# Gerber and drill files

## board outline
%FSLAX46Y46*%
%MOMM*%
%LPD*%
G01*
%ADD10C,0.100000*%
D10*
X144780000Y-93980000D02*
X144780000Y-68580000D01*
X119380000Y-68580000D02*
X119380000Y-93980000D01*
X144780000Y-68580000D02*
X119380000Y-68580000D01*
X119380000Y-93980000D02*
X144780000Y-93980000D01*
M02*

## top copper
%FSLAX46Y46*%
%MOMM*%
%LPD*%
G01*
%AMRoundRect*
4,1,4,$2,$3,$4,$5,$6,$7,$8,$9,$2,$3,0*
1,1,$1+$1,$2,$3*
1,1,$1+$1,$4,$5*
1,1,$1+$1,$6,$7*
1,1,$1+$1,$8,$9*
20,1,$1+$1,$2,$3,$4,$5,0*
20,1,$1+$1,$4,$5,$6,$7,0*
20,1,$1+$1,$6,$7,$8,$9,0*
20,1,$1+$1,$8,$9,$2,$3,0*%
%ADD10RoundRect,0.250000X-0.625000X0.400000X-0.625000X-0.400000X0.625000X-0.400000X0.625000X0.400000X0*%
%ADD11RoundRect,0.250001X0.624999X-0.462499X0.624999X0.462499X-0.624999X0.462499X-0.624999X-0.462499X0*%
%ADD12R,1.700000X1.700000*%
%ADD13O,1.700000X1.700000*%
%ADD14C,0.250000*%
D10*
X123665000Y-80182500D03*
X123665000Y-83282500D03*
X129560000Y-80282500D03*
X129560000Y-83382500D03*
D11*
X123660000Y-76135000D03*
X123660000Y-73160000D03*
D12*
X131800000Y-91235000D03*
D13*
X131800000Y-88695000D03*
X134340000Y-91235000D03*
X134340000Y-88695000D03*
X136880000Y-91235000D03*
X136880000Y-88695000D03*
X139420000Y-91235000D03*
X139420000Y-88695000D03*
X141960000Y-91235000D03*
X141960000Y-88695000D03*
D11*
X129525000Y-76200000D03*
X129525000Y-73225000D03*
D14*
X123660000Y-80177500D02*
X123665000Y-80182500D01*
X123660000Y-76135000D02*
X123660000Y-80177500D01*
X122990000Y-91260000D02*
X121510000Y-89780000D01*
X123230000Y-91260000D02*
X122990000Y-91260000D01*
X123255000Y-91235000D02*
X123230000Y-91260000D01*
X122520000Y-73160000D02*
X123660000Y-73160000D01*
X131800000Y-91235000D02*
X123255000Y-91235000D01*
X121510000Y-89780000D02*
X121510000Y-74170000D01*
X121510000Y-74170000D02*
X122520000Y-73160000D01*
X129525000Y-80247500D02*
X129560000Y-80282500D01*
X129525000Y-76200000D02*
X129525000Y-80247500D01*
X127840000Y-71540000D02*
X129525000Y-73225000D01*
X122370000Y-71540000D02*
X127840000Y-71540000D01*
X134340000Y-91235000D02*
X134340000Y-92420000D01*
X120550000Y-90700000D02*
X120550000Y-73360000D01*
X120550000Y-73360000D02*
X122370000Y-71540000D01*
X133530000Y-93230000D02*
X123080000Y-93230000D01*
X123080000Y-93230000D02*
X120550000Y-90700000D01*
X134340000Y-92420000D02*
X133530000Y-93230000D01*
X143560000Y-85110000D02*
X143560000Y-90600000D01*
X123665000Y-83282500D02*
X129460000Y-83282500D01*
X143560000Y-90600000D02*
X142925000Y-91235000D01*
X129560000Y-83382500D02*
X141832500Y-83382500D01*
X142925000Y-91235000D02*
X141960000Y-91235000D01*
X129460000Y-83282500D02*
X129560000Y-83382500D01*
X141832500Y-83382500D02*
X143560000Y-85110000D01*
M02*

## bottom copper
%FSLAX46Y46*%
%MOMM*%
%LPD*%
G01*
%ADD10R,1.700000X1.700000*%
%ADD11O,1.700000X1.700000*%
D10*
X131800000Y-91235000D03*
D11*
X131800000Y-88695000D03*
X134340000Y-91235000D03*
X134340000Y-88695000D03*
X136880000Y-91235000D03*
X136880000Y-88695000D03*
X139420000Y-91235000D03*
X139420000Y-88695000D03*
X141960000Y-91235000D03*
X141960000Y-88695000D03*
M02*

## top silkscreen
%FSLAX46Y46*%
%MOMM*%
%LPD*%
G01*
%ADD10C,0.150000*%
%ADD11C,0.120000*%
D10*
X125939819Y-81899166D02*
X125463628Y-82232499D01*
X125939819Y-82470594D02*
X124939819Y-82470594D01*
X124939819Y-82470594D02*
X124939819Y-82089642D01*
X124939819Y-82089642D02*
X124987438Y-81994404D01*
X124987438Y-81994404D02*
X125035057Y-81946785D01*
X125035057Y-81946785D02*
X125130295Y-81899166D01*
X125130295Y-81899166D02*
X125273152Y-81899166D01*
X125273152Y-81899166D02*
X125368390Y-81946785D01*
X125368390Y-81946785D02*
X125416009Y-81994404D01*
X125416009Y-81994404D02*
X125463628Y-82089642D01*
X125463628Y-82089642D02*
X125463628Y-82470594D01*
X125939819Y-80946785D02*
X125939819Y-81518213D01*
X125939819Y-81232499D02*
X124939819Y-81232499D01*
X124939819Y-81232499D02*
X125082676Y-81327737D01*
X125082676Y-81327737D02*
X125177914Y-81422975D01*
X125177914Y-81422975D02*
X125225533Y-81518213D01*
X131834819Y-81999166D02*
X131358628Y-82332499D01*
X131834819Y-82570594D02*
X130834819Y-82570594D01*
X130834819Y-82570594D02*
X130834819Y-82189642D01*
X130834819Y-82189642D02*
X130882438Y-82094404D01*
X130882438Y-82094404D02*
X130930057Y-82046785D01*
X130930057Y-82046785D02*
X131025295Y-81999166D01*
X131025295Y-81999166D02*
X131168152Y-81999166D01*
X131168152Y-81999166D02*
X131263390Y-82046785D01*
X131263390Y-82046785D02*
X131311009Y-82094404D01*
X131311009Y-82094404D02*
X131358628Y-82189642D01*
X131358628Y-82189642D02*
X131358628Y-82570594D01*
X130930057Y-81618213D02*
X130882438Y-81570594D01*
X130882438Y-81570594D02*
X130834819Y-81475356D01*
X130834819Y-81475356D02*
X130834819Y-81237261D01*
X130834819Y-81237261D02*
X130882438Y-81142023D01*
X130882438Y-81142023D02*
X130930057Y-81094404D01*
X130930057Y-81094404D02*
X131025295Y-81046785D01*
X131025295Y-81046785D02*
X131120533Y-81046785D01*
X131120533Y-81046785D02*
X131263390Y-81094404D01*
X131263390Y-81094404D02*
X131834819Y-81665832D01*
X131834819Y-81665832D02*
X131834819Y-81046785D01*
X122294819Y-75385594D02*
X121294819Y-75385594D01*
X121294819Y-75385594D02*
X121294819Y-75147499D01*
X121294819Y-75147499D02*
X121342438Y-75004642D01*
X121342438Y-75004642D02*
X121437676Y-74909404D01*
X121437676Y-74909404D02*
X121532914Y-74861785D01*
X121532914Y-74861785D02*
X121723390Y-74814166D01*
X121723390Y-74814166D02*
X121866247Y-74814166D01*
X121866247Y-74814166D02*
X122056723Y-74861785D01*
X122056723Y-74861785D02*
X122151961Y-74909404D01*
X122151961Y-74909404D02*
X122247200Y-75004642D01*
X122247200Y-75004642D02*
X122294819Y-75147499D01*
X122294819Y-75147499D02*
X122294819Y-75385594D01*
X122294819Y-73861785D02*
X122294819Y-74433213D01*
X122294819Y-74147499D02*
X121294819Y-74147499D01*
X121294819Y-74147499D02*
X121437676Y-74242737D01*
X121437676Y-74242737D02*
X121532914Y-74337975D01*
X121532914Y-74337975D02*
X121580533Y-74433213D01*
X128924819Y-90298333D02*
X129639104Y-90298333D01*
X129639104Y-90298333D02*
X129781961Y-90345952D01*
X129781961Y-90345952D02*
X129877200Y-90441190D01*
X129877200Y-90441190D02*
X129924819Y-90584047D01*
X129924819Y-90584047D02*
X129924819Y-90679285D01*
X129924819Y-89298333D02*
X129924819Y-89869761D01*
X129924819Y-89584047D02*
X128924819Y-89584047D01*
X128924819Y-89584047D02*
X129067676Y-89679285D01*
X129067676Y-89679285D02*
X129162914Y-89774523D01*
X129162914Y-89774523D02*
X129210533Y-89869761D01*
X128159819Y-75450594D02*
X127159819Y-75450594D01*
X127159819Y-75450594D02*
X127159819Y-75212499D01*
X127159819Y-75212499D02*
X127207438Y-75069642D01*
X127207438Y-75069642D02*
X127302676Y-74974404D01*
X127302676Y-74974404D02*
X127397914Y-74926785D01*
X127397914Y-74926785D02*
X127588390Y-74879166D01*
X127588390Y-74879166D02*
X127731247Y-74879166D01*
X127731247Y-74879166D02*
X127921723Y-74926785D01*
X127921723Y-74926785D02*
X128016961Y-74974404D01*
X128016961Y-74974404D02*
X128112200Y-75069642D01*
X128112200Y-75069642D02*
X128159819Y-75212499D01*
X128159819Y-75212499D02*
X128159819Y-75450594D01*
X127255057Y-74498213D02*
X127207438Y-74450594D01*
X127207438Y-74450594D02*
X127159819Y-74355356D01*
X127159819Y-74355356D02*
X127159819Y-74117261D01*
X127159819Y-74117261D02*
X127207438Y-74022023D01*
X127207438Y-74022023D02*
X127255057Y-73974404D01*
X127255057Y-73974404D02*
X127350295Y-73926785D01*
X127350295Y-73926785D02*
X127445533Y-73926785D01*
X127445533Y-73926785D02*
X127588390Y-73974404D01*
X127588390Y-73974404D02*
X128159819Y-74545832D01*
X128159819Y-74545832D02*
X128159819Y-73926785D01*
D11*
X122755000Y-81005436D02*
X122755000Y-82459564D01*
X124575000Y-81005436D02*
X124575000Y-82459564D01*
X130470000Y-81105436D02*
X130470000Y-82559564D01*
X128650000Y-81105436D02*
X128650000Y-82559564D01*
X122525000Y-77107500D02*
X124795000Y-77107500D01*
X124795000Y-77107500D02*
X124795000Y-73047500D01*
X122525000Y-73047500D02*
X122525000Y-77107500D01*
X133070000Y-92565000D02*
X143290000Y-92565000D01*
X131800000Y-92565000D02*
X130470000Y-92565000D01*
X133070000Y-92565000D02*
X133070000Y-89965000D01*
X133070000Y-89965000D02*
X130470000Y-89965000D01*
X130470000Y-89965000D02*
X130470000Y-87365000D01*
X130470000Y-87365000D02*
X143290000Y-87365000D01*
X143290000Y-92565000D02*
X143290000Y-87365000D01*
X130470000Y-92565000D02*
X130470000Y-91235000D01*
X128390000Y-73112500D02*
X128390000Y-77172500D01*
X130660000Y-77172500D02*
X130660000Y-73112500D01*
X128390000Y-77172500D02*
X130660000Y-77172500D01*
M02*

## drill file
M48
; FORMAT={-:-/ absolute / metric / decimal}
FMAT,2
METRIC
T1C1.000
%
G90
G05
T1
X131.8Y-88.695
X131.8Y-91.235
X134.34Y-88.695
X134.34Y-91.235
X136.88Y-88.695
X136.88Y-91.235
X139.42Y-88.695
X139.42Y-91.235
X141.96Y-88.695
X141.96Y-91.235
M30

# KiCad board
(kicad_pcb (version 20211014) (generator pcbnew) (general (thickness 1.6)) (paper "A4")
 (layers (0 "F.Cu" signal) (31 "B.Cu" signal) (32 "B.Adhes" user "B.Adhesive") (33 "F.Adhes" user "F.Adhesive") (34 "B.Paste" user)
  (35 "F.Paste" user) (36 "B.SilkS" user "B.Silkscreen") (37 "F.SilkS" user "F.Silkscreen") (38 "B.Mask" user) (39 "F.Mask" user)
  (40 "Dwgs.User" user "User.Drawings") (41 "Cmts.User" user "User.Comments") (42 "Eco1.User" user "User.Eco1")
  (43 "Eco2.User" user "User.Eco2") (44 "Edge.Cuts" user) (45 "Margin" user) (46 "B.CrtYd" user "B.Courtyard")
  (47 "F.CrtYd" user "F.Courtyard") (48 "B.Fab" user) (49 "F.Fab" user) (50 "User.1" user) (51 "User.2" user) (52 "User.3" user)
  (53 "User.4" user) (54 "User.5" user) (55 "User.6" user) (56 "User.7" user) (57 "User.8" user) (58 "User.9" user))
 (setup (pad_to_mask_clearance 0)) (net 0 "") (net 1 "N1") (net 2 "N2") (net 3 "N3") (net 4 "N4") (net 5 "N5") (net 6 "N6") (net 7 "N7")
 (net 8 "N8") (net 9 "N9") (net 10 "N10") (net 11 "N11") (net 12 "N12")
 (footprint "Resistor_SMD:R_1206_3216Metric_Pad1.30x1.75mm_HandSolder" (layer "F.Cu") (at 123.665 81.7325 -90)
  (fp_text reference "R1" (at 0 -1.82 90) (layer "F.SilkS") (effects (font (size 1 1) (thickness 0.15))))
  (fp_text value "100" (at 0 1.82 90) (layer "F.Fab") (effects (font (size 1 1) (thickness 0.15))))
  (fp_line (start -0.727064 0.91) (end 0.727064 0.91) (layer "F.SilkS") (width 0.12))
  (fp_line (start -0.727064 -0.91) (end 0.727064 -0.91) (layer "F.SilkS") (width 0.12))
  (pad "1" smd roundrect (at -1.55 0 270) (size 1.3 1.75) (layers "F.Cu" "F.Paste" "F.Mask") (roundrect_rratio 0.192308) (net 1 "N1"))
  (pad "2" smd roundrect (at 1.55 0 270) (size 1.3 1.75) (layers "F.Cu" "F.Paste" "F.Mask") (roundrect_rratio 0.192308) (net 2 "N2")))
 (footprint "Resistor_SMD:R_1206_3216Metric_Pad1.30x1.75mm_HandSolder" (layer "F.Cu") (at 129.56 81.8325 -90)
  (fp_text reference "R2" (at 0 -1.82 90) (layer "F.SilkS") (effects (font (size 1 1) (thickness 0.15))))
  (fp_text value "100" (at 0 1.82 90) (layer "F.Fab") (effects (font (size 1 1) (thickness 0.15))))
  (fp_line (start -0.727064 -0.91) (end 0.727064 -0.91) (layer "F.SilkS") (width 0.12))
  (fp_line (start -0.727064 0.91) (end 0.727064 0.91) (layer "F.SilkS") (width 0.12))
  (pad "1" smd roundrect (at -1.55 0 270) (size 1.3 1.75) (layers "F.Cu" "F.Paste" "F.Mask") (roundrect_rratio 0.192308) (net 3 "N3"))
  (pad "2" smd roundrect (at 1.55 0 270) (size 1.3 1.75) (layers "F.Cu" "F.Paste" "F.Mask") (roundrect_rratio 0.192308) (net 2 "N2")))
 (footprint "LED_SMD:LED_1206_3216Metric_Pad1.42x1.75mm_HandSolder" (layer "F.Cu") (at 123.66 74.6475 90)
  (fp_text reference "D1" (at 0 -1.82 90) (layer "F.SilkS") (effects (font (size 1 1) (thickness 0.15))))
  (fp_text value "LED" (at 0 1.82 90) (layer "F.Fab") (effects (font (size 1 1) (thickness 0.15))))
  (fp_line (start -2.46 -1.135) (end -2.46 1.135) (layer "F.SilkS") (width 0.12))
  (fp_line (start -2.46 1.135) (end 1.6 1.135) (layer "F.SilkS") (width 0.12))
  (fp_line (start 1.6 -1.135) (end -2.46 -1.135) (layer "F.SilkS") (width 0.12))
  (pad "1" smd roundrect (at -1.4875 0 90) (size 1.425 1.75) (layers "F.Cu" "F.Paste" "F.Mask") (roundrect_rratio 0.175439) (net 1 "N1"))
  (pad "2" smd roundrect (at 1.4875 0 90) (size 1.425 1.75) (layers "F.Cu" "F.Paste" "F.Mask") (roundrect_rratio 0.175439) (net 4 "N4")))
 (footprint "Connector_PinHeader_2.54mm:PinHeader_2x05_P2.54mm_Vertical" (layer "F.Cu") (at 131.8 91.235 90)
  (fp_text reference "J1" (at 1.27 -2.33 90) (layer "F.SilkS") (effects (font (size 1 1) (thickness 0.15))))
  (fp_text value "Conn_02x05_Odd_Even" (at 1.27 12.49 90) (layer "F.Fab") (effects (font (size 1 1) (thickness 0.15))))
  (fp_line (start -1.33 1.27) (end -1.33 11.49) (layer "F.SilkS") (width 0.12))
  (fp_line (start -1.33 0) (end -1.33 -1.33) (layer "F.SilkS") (width 0.12))
  (fp_line (start -1.33 1.27) (end 1.27 1.27) (layer "F.SilkS") (width 0.12))
  (fp_line (start 1.27 1.27) (end 1.27 -1.33) (layer "F.SilkS") (width 0.12))
  (fp_line (start 1.27 -1.33) (end 3.87 -1.33) (layer "F.SilkS") (width 0.12))
  (fp_line (start 3.87 -1.33) (end 3.87 11.49) (layer "F.SilkS") (width 0.12))
  (fp_line (start -1.33 11.49) (end 3.87 11.49) (layer "F.SilkS") (width 0.12))
  (fp_line (start -1.33 -1.33) (end 0 -1.33) (layer "F.SilkS") (width 0.12))
  (pad "1" thru_hole rect (at 0 0 90) (size 1.7 1.7) (drill 1) (layers *.Cu *.Mask) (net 4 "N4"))
  (pad "2" thru_hole oval (at 2.54 0 90) (size 1.7 1.7) (drill 1) (layers *.Cu *.Mask) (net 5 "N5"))
  (pad "3" thru_hole oval (at 0 2.54 90) (size 1.7 1.7) (drill 1) (layers *.Cu *.Mask) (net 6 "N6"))
  (pad "4" thru_hole oval (at 2.54 2.54 90) (size 1.7 1.7) (drill 1) (layers *.Cu *.Mask) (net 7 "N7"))
  (pad "5" thru_hole oval (at 0 5.08 90) (size 1.7 1.7) (drill 1) (layers *.Cu *.Mask) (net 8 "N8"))
  (pad "6" thru_hole oval (at 2.54 5.08 90) (size 1.7 1.7) (drill 1) (layers *.Cu *.Mask) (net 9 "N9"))
  (pad "7" thru_hole oval (at 0 7.62 90) (size 1.7 1.7) (drill 1) (layers *.Cu *.Mask) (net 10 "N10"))
  (pad "8" thru_hole oval (at 2.54 7.62 90) (size 1.7 1.7) (drill 1) (layers *.Cu *.Mask) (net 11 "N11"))
  (pad "9" thru_hole oval (at 0 10.16 90) (size 1.7 1.7) (drill 1) (layers *.Cu *.Mask) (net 2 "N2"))
  (pad "10" thru_hole oval (at 2.54 10.16 90) (size 1.7 1.7) (drill 1) (layers *.Cu *.Mask) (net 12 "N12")))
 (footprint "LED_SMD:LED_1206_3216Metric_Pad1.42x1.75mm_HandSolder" (layer "F.Cu") (at 129.525 74.7125 90)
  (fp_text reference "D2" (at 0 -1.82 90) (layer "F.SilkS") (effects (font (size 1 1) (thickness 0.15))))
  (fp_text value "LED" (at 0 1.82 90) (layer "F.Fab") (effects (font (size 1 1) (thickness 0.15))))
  (fp_line (start 1.6 -1.135) (end -2.46 -1.135) (layer "F.SilkS") (width 0.12))
  (fp_line (start -2.46 1.135) (end 1.6 1.135) (layer "F.SilkS") (width 0.12))
  (fp_line (start -2.46 -1.135) (end -2.46 1.135) (layer "F.SilkS") (width 0.12))
  (pad "1" smd roundrect (at -1.4875 0 90) (size 1.425 1.75) (layers "F.Cu" "F.Paste" "F.Mask") (roundrect_rratio 0.175439) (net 3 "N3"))
  (pad "2" smd roundrect (at 1.4875 0 90) (size 1.425 1.75) (layers "F.Cu" "F.Paste" "F.Mask") (roundrect_rratio 0.175439) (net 6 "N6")))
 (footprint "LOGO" (layer "B.Cu") (at 132.12 79.85 180)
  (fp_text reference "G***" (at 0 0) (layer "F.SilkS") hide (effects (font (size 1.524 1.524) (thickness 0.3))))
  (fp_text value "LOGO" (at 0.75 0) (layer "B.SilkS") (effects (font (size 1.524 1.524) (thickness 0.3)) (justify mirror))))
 (gr_line (start 144.78 93.98) (end 144.78 68.58) (layer "Edge.Cuts") (width 0.1))
 (gr_line (start 119.38 68.58) (end 119.38 93.98) (layer "Edge.Cuts") (width 0.1))
 (gr_line (start 144.78 68.58) (end 119.38 68.58) (layer "Edge.Cuts") (width 0.1))
 (gr_line (start 119.38 93.98) (end 144.78 93.98) (layer "Edge.Cuts") (width 0.1))
 (segment (start 123.66 80.1775) (end 123.665 80.1825) (width 0.25) (layer "F.Cu") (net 1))
 (segment (start 123.66 76.135) (end 123.66 80.1775) (width 0.25) (layer "F.Cu") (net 1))
 (segment (start 122.99 91.26) (end 121.51 89.78) (width 0.25) (layer "F.Cu") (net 4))
 (segment (start 123.23 91.26) (end 122.99 91.26) (width 0.25) (layer "F.Cu") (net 4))
 (segment (start 123.255 91.235) (end 123.23 91.26) (width 0.25) (layer "F.Cu") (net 4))
 (segment (start 122.52 73.16) (end 123.66 73.16) (width 0.25) (layer "F.Cu") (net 4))
 (segment (start 131.8 91.235) (end 123.255 91.235) (width 0.25) (layer "F.Cu") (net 4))
 (segment (start 121.51 89.78) (end 121.51 74.17) (width 0.25) (layer "F.Cu") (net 4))
 (segment (start 121.51 74.17) (end 122.52 73.16) (width 0.25) (layer "F.Cu") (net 4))
 (segment (start 129.525 80.2475) (end 129.56 80.2825) (width 0.25) (layer "F.Cu") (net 3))
 (segment (start 129.525 76.2) (end 129.525 80.2475) (width 0.25) (layer "F.Cu") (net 3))
 (segment (start 127.84 71.54) (end 129.525 73.225) (width 0.25) (layer "F.Cu") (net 6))
 (segment (start 122.37 71.54) (end 127.84 71.54) (width 0.25) (layer "F.Cu") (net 6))
 (segment (start 134.34 91.235) (end 134.34 92.42) (width 0.25) (layer "F.Cu") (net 6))
 (segment (start 120.55 90.7) (end 120.55 73.36) (width 0.25) (layer "F.Cu") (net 6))
 (segment (start 120.55 73.36) (end 122.37 71.54) (width 0.25) (layer "F.Cu") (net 6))
 (segment (start 133.53 93.23) (end 123.08 93.23) (width 0.25) (layer "F.Cu") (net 6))
 (segment (start 123.08 93.23) (end 120.55 90.7) (width 0.25) (layer "F.Cu") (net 6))
 (segment (start 134.34 92.42) (end 133.53 93.23) (width 0.25) (layer "F.Cu") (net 6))
 (segment (start 143.56 85.11) (end 143.56 90.6) (width 0.25) (layer "F.Cu") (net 2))
 (segment (start 123.665 83.2825) (end 129.46 83.2825) (width 0.25) (layer "F.Cu") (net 2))
 (segment (start 143.56 90.6) (end 142.925 91.235) (width 0.25) (layer "F.Cu") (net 2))
 (segment (start 129.56 83.3825) (end 141.8325 83.3825) (width 0.25) (layer "F.Cu") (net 2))
 (segment (start 142.925 91.235) (end 141.96 91.235) (width 0.25) (layer "F.Cu") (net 2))
 (segment (start 129.46 83.2825) (end 129.56 83.3825) (width 0.25) (layer "F.Cu") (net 2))
 (segment (start 141.8325 83.3825) (end 143.56 85.11) (width 0.25) (layer "F.Cu") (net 2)))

